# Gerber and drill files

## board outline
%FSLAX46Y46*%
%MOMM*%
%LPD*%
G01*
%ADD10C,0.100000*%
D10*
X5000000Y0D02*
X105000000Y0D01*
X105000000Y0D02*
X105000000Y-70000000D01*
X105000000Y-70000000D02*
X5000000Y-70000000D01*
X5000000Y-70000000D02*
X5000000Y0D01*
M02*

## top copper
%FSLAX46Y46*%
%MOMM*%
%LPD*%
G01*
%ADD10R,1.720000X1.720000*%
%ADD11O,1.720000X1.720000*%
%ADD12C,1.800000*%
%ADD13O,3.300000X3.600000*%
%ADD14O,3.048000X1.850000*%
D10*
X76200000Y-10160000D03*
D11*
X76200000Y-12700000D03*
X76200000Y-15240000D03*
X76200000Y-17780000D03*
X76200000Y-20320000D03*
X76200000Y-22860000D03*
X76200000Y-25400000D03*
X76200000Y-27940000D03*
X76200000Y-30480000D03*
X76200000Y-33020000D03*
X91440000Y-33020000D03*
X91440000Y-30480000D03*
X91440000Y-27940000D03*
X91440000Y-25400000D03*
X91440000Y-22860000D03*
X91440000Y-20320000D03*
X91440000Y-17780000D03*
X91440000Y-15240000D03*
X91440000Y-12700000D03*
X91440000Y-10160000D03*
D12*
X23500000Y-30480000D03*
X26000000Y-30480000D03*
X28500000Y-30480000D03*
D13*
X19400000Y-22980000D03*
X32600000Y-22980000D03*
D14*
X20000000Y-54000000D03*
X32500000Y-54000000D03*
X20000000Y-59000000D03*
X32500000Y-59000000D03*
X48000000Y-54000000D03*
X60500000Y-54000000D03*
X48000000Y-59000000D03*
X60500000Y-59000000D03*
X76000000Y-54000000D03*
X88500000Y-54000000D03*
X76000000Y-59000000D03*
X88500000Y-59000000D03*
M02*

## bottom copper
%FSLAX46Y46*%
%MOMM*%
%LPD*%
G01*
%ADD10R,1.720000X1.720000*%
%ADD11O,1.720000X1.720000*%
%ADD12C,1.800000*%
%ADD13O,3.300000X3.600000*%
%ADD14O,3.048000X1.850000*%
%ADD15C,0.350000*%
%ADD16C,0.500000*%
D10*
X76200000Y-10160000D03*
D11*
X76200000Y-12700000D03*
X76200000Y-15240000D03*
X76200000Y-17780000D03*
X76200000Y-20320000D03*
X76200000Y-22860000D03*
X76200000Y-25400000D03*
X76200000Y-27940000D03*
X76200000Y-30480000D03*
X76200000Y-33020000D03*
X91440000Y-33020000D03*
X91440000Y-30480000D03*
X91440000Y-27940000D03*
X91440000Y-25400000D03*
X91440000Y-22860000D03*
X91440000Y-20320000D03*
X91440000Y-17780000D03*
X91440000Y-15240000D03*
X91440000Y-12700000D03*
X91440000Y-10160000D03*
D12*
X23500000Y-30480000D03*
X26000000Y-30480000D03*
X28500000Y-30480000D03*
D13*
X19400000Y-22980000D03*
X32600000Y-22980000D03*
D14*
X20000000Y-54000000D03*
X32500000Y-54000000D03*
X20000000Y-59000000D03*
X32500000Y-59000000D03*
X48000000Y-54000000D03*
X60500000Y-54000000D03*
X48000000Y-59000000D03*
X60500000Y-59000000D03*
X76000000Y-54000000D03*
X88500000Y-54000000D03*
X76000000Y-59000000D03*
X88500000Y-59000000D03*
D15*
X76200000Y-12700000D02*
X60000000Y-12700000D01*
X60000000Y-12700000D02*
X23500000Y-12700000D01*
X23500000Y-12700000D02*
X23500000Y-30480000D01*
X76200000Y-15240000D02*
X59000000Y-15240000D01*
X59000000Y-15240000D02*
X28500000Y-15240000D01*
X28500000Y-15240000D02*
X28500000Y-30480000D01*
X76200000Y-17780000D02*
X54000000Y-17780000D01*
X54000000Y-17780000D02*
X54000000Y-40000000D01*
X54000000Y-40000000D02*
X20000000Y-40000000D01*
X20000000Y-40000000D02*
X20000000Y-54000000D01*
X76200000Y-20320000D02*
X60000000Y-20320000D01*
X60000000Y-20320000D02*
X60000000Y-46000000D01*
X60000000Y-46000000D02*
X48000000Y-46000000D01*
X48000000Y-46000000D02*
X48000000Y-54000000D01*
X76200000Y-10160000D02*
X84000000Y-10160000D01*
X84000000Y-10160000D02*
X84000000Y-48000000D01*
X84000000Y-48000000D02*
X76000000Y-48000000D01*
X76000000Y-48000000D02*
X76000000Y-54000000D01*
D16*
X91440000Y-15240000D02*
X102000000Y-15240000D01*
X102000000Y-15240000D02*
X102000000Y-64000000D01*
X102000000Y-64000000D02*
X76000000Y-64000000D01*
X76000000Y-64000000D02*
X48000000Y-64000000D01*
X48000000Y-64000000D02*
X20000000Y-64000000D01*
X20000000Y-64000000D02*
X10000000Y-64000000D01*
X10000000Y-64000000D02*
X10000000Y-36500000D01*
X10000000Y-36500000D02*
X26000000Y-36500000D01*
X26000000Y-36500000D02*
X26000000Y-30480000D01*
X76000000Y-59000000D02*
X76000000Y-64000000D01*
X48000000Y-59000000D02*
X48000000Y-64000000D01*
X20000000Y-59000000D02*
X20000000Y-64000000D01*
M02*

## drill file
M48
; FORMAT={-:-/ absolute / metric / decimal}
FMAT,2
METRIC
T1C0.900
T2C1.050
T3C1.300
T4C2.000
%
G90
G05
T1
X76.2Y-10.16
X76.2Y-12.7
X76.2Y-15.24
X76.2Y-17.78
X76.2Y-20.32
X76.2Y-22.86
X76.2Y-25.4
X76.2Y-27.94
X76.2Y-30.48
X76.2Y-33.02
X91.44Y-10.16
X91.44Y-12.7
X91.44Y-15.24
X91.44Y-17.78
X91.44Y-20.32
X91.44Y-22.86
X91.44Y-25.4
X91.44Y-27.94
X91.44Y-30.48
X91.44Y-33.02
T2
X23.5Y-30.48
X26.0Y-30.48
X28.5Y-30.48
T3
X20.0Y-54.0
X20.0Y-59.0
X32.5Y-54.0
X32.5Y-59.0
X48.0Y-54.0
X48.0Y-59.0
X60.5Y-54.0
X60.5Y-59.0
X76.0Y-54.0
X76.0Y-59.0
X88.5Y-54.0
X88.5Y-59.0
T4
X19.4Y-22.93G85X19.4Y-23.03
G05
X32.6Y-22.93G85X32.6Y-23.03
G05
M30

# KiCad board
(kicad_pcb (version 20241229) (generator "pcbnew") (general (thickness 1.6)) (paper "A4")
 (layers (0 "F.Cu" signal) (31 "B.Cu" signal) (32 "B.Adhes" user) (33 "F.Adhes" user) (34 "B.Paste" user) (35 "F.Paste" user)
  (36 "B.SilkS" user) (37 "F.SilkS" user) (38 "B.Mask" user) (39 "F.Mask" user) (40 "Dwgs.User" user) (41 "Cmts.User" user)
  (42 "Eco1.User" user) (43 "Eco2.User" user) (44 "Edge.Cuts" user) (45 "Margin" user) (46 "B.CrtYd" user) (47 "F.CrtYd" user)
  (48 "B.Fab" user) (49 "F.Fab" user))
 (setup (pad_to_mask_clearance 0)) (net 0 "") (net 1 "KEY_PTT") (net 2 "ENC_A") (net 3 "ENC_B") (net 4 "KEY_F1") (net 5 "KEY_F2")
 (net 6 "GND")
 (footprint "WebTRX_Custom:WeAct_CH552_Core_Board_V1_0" (layer "F.Cu") (at 76.2 10.16)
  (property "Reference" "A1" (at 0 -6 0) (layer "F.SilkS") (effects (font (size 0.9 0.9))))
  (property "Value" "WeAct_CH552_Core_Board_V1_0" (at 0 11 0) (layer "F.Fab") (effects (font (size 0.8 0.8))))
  (pad "1" thru_hole rect (at 0 0) (size 1.72 1.72) (drill 0.9) (layers "*.Cu" "*.Mask") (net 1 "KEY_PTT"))
  (pad "2" thru_hole oval (at 0 2.54) (size 1.72 1.72) (drill 0.9) (layers "*.Cu" "*.Mask") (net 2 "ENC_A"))
  (pad "3" thru_hole oval (at 0 5.08) (size 1.72 1.72) (drill 0.9) (layers "*.Cu" "*.Mask") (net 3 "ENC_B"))
  (pad "4" thru_hole oval (at 0 7.62) (size 1.72 1.72) (drill 0.9) (layers "*.Cu" "*.Mask") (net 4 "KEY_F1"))
  (pad "5" thru_hole oval (at 0 10.16) (size 1.72 1.72) (drill 0.9) (layers "*.Cu" "*.Mask") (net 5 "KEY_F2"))
  (pad "6" thru_hole oval (at 0 12.7) (size 1.72 1.72) (drill 0.9) (layers "*.Cu" "*.Mask"))
  (pad "7" thru_hole oval (at 0 15.24) (size 1.72 1.72) (drill 0.9) (layers "*.Cu" "*.Mask"))
  (pad "8" thru_hole oval (at 0 17.78) (size 1.72 1.72) (drill 0.9) (layers "*.Cu" "*.Mask"))
  (pad "9" thru_hole oval (at 0 20.32) (size 1.72 1.72) (drill 0.9) (layers "*.Cu" "*.Mask"))
  (pad "10" thru_hole oval (at 0 22.86) (size 1.72 1.72) (drill 0.9) (layers "*.Cu" "*.Mask"))
  (pad "11" thru_hole oval (at 15.24 22.86) (size 1.72 1.72) (drill 0.9) (layers "*.Cu" "*.Mask"))
  (pad "12" thru_hole oval (at 15.24 20.32) (size 1.72 1.72) (drill 0.9) (layers "*.Cu" "*.Mask"))
  (pad "13" thru_hole oval (at 15.24 17.78) (size 1.72 1.72) (drill 0.9) (layers "*.Cu" "*.Mask"))
  (pad "14" thru_hole oval (at 15.24 15.24) (size 1.72 1.72) (drill 0.9) (layers "*.Cu" "*.Mask"))
  (pad "15" thru_hole oval (at 15.24 12.7) (size 1.72 1.72) (drill 0.9) (layers "*.Cu" "*.Mask"))
  (pad "16" thru_hole oval (at 15.24 10.16) (size 1.72 1.72) (drill 0.9) (layers "*.Cu" "*.Mask"))
  (pad "17" thru_hole oval (at 15.24 7.62) (size 1.72 1.72) (drill 0.9) (layers "*.Cu" "*.Mask"))
  (pad "18" thru_hole oval (at 15.24 5.08) (size 1.72 1.72) (drill 0.9) (layers "*.Cu" "*.Mask") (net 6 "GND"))
  (pad "19" thru_hole oval (at 15.24 2.54) (size 1.72 1.72) (drill 0.9) (layers "*.Cu" "*.Mask"))
  (pad "20" thru_hole oval (at 15.24 0) (size 1.72 1.72) (drill 0.9) (layers "*.Cu" "*.Mask")))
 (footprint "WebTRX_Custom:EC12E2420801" (layer "F.Cu") (at 26 30.48)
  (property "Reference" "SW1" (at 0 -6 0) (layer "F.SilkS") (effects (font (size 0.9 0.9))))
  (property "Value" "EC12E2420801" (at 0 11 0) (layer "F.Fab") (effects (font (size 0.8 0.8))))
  (pad "A" thru_hole circle (at -2.5 0) (size 1.8 1.8) (drill 1.05) (layers "*.Cu" "*.Mask") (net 2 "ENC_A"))
  (pad "C" thru_hole circle (at 0 0) (size 1.8 1.8) (drill 1.05) (layers "*.Cu" "*.Mask") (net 6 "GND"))
  (pad "B" thru_hole circle (at 2.5 0) (size 1.8 1.8) (drill 1.05) (layers "*.Cu" "*.Mask") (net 3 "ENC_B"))
  (pad "M1" thru_hole oval (at -6.6 -7.5) (size 3.3 3.6) (drill oval 2 2.1) (layers "*.Cu" "*.Mask"))
  (pad "M2" thru_hole oval (at 6.6 -7.5) (size 3.3 3.6) (drill oval 2 2.1) (layers "*.Cu" "*.Mask")))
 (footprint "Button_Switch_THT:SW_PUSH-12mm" (layer "F.Cu") (at 20 54)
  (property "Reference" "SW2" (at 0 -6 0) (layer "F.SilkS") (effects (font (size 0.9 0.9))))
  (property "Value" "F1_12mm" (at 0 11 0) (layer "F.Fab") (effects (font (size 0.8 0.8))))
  (pad "1" thru_hole oval (at 0 0) (size 3.048 1.85) (drill 1.3) (layers "*.Cu" "*.Mask") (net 4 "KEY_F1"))
  (pad "1" thru_hole oval (at 12.5 0) (size 3.048 1.85) (drill 1.3) (layers "*.Cu" "*.Mask") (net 4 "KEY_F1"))
  (pad "2" thru_hole oval (at 0 5) (size 3.048 1.85) (drill 1.3) (layers "*.Cu" "*.Mask") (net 6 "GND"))
  (pad "2" thru_hole oval (at 12.5 5) (size 3.048 1.85) (drill 1.3) (layers "*.Cu" "*.Mask") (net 6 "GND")))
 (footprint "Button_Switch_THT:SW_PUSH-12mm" (layer "F.Cu") (at 48 54)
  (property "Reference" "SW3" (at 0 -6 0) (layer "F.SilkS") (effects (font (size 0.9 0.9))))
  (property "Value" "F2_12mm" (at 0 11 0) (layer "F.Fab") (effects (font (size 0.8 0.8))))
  (pad "1" thru_hole oval (at 0 0) (size 3.048 1.85) (drill 1.3) (layers "*.Cu" "*.Mask") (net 5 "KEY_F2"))
  (pad "1" thru_hole oval (at 12.5 0) (size 3.048 1.85) (drill 1.3) (layers "*.Cu" "*.Mask") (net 5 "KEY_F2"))
  (pad "2" thru_hole oval (at 0 5) (size 3.048 1.85) (drill 1.3) (layers "*.Cu" "*.Mask") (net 6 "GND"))
  (pad "2" thru_hole oval (at 12.5 5) (size 3.048 1.85) (drill 1.3) (layers "*.Cu" "*.Mask") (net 6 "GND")))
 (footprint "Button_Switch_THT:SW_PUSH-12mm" (layer "F.Cu") (at 76 54)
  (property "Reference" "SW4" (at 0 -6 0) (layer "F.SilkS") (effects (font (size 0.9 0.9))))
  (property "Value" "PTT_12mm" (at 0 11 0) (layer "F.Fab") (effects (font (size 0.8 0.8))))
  (pad "1" thru_hole oval (at 0 0) (size 3.048 1.85) (drill 1.3) (layers "*.Cu" "*.Mask") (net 1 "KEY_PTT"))
  (pad "1" thru_hole oval (at 12.5 0) (size 3.048 1.85) (drill 1.3) (layers "*.Cu" "*.Mask") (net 1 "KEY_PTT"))
  (pad "2" thru_hole oval (at 0 5) (size 3.048 1.85) (drill 1.3) (layers "*.Cu" "*.Mask") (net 6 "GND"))
  (pad "2" thru_hole oval (at 12.5 5) (size 3.048 1.85) (drill 1.3) (layers "*.Cu" "*.Mask") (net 6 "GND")))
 (gr_line (start 5 0) (end 105 0) (stroke (width 0.1) (type default)) (layer "Edge.Cuts"))
 (gr_line (start 105 0) (end 105 70) (stroke (width 0.1) (type default)) (layer "Edge.Cuts"))
 (gr_line (start 105 70) (end 5 70) (stroke (width 0.1) (type default)) (layer "Edge.Cuts"))
 (gr_line (start 5 70) (end 5 0) (stroke (width 0.1) (type default)) (layer "Edge.Cuts"))
 (segment (start 76.2 12.7) (end 60 12.7) (width 0.35) (layer "B.Cu") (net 2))
 (segment (start 60 12.7) (end 23.5 12.7) (width 0.35) (layer "B.Cu") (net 2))
 (segment (start 23.5 12.7) (end 23.5 30.48) (width 0.35) (layer "B.Cu") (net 2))
 (segment (start 76.2 15.24) (end 59 15.24) (width 0.35) (layer "B.Cu") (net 3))
 (segment (start 59 15.24) (end 28.5 15.24) (width 0.35) (layer "B.Cu") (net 3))
 (segment (start 28.5 15.24) (end 28.5 30.48) (width 0.35) (layer "B.Cu") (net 3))
 (segment (start 76.2 17.78) (end 54 17.78) (width 0.35) (layer "B.Cu") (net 4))
 (segment (start 54 17.78) (end 54 40) (width 0.35) (layer "B.Cu") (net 4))
 (segment (start 54 40) (end 20 40) (width 0.35) (layer "B.Cu") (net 4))
 (segment (start 20 40) (end 20 54) (width 0.35) (layer "B.Cu") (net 4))
 (segment (start 76.2 20.32) (end 60 20.32) (width 0.35) (layer "B.Cu") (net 5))
 (segment (start 60 20.32) (end 60 46) (width 0.35) (layer "B.Cu") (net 5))
 (segment (start 60 46) (end 48 46) (width 0.35) (layer "B.Cu") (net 5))
 (segment (start 48 46) (end 48 54) (width 0.35) (layer "B.Cu") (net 5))
 (segment (start 76.2 10.16) (end 84 10.16) (width 0.35) (layer "B.Cu") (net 1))
 (segment (start 84 10.16) (end 84 48) (width 0.35) (layer "B.Cu") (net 1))
 (segment (start 84 48) (end 76 48) (width 0.35) (layer "B.Cu") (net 1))
 (segment (start 76 48) (end 76 54) (width 0.35) (layer "B.Cu") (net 1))
 (segment (start 91.44 15.24) (end 102 15.24) (width 0.5) (layer "B.Cu") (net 6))
 (segment (start 102 15.24) (end 102 64) (width 0.5) (layer "B.Cu") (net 6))
 (segment (start 102 64) (end 76 64) (width 0.5) (layer "B.Cu") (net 6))
 (segment (start 76 64) (end 48 64) (width 0.5) (layer "B.Cu") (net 6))
 (segment (start 48 64) (end 20 64) (width 0.5) (layer "B.Cu") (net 6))
 (segment (start 20 64) (end 10 64) (width 0.5) (layer "B.Cu") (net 6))
 (segment (start 10 64) (end 10 36.5) (width 0.5) (layer "B.Cu") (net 6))
 (segment (start 10 36.5) (end 26 36.5) (width 0.5) (layer "B.Cu") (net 6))
 (segment (start 26 36.5) (end 26 30.48) (width 0.5) (layer "B.Cu") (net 6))
 (segment (start 76 59) (end 76 64) (width 0.5) (layer "B.Cu") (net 6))
 (segment (start 48 59) (end 48 64) (width 0.5) (layer "B.Cu") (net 6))
 (segment (start 20 59) (end 20 64) (width 0.5) (layer "B.Cu") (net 6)))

